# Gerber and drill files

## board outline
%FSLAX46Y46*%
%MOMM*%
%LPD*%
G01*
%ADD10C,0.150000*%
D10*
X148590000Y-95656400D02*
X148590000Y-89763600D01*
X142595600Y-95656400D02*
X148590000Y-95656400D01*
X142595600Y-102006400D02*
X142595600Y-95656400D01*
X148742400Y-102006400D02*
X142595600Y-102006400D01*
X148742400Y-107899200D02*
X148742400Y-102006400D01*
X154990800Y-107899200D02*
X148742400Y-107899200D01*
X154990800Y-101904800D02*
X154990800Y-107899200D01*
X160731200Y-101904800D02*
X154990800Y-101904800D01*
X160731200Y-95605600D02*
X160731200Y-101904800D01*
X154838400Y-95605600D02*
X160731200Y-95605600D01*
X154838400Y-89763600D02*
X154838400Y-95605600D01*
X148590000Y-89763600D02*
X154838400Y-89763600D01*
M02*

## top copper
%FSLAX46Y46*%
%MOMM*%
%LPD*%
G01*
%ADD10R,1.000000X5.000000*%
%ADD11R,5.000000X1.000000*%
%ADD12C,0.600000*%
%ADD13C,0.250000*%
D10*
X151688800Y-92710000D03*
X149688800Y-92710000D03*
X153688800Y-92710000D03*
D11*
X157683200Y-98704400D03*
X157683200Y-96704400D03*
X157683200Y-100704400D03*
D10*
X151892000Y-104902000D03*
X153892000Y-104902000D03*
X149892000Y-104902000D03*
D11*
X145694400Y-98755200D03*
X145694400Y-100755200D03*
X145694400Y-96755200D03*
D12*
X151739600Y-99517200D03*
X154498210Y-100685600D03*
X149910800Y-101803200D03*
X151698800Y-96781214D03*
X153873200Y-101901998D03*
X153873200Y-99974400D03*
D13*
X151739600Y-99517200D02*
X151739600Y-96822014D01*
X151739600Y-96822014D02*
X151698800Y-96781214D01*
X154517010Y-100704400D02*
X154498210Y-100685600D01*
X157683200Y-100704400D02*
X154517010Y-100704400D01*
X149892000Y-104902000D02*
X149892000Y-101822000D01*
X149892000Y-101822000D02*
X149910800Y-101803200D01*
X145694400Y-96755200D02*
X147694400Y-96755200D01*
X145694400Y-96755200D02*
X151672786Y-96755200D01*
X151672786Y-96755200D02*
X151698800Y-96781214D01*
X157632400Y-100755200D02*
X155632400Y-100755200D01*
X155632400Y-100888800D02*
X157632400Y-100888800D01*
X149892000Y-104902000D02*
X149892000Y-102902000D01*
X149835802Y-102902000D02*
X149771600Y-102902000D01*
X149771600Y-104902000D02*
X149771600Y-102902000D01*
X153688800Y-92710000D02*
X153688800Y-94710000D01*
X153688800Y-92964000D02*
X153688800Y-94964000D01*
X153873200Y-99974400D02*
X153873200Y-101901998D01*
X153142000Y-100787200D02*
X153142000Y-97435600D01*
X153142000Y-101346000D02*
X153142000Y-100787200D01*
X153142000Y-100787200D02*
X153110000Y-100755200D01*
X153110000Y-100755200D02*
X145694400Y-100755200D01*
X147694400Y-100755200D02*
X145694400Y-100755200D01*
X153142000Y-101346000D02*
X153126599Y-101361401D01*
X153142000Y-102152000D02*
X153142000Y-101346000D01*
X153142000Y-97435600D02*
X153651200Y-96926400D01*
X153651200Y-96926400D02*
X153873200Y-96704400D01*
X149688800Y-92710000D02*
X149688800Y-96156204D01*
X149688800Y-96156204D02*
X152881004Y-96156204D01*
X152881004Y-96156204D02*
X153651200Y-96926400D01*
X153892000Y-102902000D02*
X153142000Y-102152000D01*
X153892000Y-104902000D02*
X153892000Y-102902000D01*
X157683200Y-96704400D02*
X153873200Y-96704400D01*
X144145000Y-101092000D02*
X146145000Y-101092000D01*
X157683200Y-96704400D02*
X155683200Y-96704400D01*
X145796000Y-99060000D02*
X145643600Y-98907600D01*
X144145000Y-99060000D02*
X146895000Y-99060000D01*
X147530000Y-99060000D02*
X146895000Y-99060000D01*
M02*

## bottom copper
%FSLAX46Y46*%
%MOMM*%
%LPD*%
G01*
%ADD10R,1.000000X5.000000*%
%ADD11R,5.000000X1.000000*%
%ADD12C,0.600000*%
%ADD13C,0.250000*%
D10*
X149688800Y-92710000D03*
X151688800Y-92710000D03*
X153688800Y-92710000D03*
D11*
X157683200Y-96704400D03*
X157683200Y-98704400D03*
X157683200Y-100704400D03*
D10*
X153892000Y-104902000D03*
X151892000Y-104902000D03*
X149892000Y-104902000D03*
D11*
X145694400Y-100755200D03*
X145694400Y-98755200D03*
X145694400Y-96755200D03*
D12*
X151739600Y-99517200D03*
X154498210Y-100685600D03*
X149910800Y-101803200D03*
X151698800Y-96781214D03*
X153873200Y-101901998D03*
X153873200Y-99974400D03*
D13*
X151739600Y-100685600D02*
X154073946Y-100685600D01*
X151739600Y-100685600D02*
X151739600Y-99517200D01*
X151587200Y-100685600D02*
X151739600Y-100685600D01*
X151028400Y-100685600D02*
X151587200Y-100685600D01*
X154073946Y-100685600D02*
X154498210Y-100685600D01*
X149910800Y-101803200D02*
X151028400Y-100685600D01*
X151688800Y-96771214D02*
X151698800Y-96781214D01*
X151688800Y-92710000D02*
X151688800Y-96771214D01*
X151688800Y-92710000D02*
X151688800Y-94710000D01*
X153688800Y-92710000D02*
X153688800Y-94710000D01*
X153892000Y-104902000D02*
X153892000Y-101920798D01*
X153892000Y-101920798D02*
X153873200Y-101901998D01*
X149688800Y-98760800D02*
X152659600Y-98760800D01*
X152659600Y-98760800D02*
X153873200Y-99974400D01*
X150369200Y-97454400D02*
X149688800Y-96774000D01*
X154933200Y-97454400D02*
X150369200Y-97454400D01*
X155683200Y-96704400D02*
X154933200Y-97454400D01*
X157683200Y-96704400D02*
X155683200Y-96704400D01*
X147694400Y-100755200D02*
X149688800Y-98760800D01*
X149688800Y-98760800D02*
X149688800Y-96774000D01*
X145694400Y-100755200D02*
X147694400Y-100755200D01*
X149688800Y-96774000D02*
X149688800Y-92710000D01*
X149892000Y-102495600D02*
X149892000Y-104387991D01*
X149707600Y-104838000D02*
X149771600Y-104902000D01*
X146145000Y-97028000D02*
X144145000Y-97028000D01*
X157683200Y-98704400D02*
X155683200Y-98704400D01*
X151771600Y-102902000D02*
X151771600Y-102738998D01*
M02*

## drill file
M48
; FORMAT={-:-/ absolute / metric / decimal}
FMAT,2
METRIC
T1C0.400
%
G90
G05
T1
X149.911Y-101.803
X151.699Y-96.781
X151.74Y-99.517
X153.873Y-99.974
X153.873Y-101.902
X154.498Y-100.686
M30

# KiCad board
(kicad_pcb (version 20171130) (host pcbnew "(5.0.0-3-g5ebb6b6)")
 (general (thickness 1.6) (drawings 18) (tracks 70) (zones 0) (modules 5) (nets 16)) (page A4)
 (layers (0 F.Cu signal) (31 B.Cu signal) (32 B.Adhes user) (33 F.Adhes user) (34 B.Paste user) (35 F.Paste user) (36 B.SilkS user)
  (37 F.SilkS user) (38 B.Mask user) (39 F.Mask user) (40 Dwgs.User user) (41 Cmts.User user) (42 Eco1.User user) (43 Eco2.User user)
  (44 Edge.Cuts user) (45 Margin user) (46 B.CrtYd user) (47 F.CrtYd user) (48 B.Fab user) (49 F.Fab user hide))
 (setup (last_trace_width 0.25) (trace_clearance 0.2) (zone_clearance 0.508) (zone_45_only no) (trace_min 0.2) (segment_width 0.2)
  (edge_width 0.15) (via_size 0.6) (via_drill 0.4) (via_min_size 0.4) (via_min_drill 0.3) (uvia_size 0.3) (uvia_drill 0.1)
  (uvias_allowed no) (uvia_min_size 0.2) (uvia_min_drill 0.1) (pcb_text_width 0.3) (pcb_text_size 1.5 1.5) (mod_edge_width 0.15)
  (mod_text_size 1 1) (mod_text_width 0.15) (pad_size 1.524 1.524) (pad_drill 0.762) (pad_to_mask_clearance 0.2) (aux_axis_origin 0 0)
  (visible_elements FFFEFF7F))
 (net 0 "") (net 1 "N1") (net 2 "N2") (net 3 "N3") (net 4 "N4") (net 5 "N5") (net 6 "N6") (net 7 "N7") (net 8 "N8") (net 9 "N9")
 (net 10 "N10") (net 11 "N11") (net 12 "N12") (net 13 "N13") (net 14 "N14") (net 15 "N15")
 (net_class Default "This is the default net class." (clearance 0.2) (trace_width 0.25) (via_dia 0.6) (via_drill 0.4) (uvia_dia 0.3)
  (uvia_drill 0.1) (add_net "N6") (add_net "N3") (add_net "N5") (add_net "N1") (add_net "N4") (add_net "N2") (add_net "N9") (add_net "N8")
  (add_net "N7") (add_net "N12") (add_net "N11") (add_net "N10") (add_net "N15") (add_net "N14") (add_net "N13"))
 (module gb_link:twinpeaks (layer B.Cu) (at 149.86 100.33 180)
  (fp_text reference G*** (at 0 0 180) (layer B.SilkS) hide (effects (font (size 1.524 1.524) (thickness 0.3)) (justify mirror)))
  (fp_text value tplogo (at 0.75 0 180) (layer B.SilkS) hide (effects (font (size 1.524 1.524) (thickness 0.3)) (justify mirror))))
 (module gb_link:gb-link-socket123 (layer F.Cu) (at 151.6888 92.71 180)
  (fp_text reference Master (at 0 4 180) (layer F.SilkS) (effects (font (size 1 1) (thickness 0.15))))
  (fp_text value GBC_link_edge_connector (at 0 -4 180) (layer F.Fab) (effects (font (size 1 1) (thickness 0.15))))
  (pad 4 connect rect (at 0 0 180) (size 1 5) (layers F.Cu F.Mask) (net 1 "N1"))
  (pad 6 connect rect (at 2 0 180) (size 1 5) (layers F.Cu F.Mask) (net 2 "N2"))
  (pad 2 connect rect (at -2 0 180) (size 1 5) (layers F.Cu F.Mask) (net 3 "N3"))
  (pad 5 connect rect (at 2 0 180) (size 1 5) (layers B.Cu B.Mask) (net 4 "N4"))
  (pad 3 connect rect (at 0 0 180) (size 1 5) (layers B.Cu B.Mask) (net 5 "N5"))
  (pad 1 connect rect (at -2 0 180) (size 1 5) (layers B.Cu B.Mask) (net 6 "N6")))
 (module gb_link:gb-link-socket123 (layer F.Cu) (at 157.6832 98.7044 90)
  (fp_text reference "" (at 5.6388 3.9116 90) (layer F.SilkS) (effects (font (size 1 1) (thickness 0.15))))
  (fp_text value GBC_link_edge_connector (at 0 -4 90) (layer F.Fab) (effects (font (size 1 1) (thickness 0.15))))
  (pad 4 connect rect (at 0 0 90) (size 1 5) (layers F.Cu F.Mask) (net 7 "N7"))
  (pad 6 connect rect (at 2 0 90) (size 1 5) (layers F.Cu F.Mask) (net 2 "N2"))
  (pad 2 connect rect (at -2 0 90) (size 1 5) (layers F.Cu F.Mask) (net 5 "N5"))
  (pad 5 connect rect (at 2 0 90) (size 1 5) (layers B.Cu B.Mask) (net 4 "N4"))
  (pad 3 connect rect (at 0 0 90) (size 1 5) (layers B.Cu B.Mask) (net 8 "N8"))
  (pad 1 connect rect (at -2 0 90) (size 1 5) (layers B.Cu B.Mask) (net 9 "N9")))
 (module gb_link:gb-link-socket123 (layer F.Cu) (at 151.892 104.902)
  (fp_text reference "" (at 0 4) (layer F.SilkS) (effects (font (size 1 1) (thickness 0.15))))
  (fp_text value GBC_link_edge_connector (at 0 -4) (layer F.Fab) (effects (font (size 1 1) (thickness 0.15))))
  (pad 4 connect rect (at 0 0) (size 1 5) (layers F.Cu F.Mask) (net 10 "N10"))
  (pad 6 connect rect (at 2 0) (size 1 5) (layers F.Cu F.Mask) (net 2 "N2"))
  (pad 2 connect rect (at -2 0) (size 1 5) (layers F.Cu F.Mask) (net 5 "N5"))
  (pad 5 connect rect (at 2 0) (size 1 5) (layers B.Cu B.Mask) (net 4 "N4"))
  (pad 3 connect rect (at 0 0) (size 1 5) (layers B.Cu B.Mask) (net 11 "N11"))
  (pad 1 connect rect (at -2 0) (size 1 5) (layers B.Cu B.Mask) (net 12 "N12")))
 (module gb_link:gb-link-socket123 (layer F.Cu) (at 145.6944 98.7552 270)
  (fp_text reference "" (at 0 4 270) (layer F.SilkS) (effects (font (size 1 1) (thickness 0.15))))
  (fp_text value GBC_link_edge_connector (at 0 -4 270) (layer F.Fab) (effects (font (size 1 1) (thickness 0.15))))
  (pad 4 connect rect (at 0 0 270) (size 1 5) (layers F.Cu F.Mask) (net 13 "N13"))
  (pad 6 connect rect (at 2 0 270) (size 1 5) (layers F.Cu F.Mask) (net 2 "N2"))
  (pad 2 connect rect (at -2 0 270) (size 1 5) (layers F.Cu F.Mask) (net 5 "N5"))
  (pad 5 connect rect (at 2 0 270) (size 1 5) (layers B.Cu B.Mask) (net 4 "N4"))
  (pad 3 connect rect (at 0 0 270) (size 1 5) (layers B.Cu B.Mask) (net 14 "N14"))
  (pad 1 connect rect (at -2 0 270) (size 1 5) (layers B.Cu B.Mask) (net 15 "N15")))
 (gr_line (start 148.59 95.6564) (end 148.59 89.7636) (layer Edge.Cuts) (width 0.15))
 (gr_line (start 142.5956 95.6564) (end 148.59 95.6564) (layer Edge.Cuts) (width 0.15))
 (gr_line (start 142.5956 102.0064) (end 142.5956 95.6564) (layer Edge.Cuts) (width 0.15))
 (gr_line (start 148.7424 102.0064) (end 142.5956 102.0064) (layer Edge.Cuts) (width 0.15))
 (gr_line (start 148.7424 107.8992) (end 148.7424 102.0064) (layer Edge.Cuts) (width 0.15))
 (gr_line (start 154.9908 107.8992) (end 148.7424 107.8992) (layer Edge.Cuts) (width 0.15))
 (gr_line (start 154.9908 101.9048) (end 154.9908 107.8992) (layer Edge.Cuts) (width 0.15))
 (gr_line (start 160.7312 101.9048) (end 154.9908 101.9048) (layer Edge.Cuts) (width 0.15))
 (gr_line (start 160.7312 95.6056) (end 160.7312 101.9048) (layer Edge.Cuts) (width 0.15))
 (gr_line (start 154.8384 95.6056) (end 160.7312 95.6056) (layer Edge.Cuts) (width 0.15))
 (gr_line (start 154.8384 89.7636) (end 154.8384 95.6056) (layer Edge.Cuts) (width 0.15))
 (gr_line (start 148.59 89.7636) (end 154.8384 89.7636) (layer Edge.Cuts) (width 0.15))
 (segment (start 151.7396 99.5172) (end 151.7396 96.822014) (width 0.25) (layer F.Cu) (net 5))
 (segment (start 151.7396 96.822014) (end 151.6988 96.781214) (width 0.25) (layer F.Cu) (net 5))
 (segment (start 151.7396 100.6856) (end 154.073946 100.6856) (width 0.25) (layer B.Cu) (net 5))
 (segment (start 151.7396 100.6856) (end 151.7396 99.5172) (width 0.25) (layer B.Cu) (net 5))
 (segment (start 151.5872 100.6856) (end 151.7396 100.6856) (width 0.25) (layer B.Cu) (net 5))
 (via (at 151.7396 99.5172) (size 0.6) (drill 0.4) (layers F.Cu B.Cu) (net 5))
 (segment (start 151.0284 100.6856) (end 151.5872 100.6856) (width 0.25) (layer B.Cu) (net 5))
 (segment (start 154.073946 100.6856) (end 154.49821 100.6856) (width 0.25) (layer B.Cu) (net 5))
 (segment (start 149.9108 101.8032) (end 151.0284 100.6856) (width 0.25) (layer B.Cu) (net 5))
 (segment (start 154.51701 100.7044) (end 154.49821 100.6856) (width 0.25) (layer F.Cu) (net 5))
 (segment (start 157.6832 100.7044) (end 154.51701 100.7044) (width 0.25) (layer F.Cu) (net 5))
 (via (at 154.49821 100.6856) (size 0.6) (drill 0.4) (layers F.Cu B.Cu) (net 5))
 (segment (start 149.892 104.902) (end 149.892 101.822) (width 0.25) (layer F.Cu) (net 5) (status 10))
 (segment (start 149.892 101.822) (end 149.9108 101.8032) (width 0.25) (layer F.Cu) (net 5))
 (via (at 149.9108 101.8032) (size 0.6) (drill 0.4) (layers F.Cu B.Cu) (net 5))
 (segment (start 145.6944 96.7552) (end 147.6944 96.7552) (width 0.25) (layer F.Cu) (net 5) (status 30))
 (segment (start 145.6944 96.7552) (end 151.672786 96.7552) (width 0.25) (layer F.Cu) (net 5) (status 10))
 (segment (start 151.6888 96.771214) (end 151.6988 96.781214) (width 0.25) (layer B.Cu) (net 5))
 (segment (start 151.6888 92.71) (end 151.6888 96.771214) (width 0.25) (layer B.Cu) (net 5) (status 10))
 (segment (start 151.672786 96.7552) (end 151.6988 96.781214) (width 0.25) (layer F.Cu) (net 5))
 (via (at 151.6988 96.781214) (size 0.6) (drill 0.4) (layers F.Cu B.Cu) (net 5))
 (segment (start 151.6888 92.71) (end 151.6888 94.71) (width 0.25) (layer B.Cu) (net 5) (status 30))
 (segment (start 157.6324 100.7552) (end 155.6324 100.7552) (width 0.25) (layer F.Cu) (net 5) (status 30))
 (segment (start 155.6324 100.8888) (end 157.6324 100.8888) (width 0.25) (layer F.Cu) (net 5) (status 30))
 (segment (start 149.892 104.902) (end 149.892 102.902) (width 0.25) (layer F.Cu) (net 5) (status 30))
 (segment (start 149.835802 102.902) (end 149.7716 102.902) (width 0.25) (layer F.Cu) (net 5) (status 30))
 (segment (start 149.7716 104.902) (end 149.7716 102.902) (width 0.25) (layer F.Cu) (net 5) (status 30))
 (segment (start 153.6888 92.71) (end 153.6888 94.71) (width 0.25) (layer B.Cu) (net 6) (status 30))
 (segment (start 153.6888 92.71) (end 153.6888 94.71) (width 0.25) (layer F.Cu) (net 3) (status 30))
 (segment (start 153.6888 92.964) (end 153.6888 94.964) (width 0.25) (layer F.Cu) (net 3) (status 30))
 (segment (start 153.892 104.902) (end 153.892 101.920798) (width 0.25) (layer B.Cu) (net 4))
 (segment (start 153.892 101.920798) (end 153.8732 101.901998) (width 0.25) (layer B.Cu) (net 4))
 (segment (start 153.8732 99.9744) (end 153.8732 101.901998) (width 0.25) (layer F.Cu) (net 4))
 (via (at 153.8732 101.901998) (size 0.6) (drill 0.4) (layers F.Cu B.Cu) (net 4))
 (via (at 153.8732 99.9744) (size 0.6) (drill 0.4) (layers F.Cu B.Cu) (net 4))
 (segment (start 149.6888 98.7608) (end 152.6596 98.7608) (width 0.25) (layer B.Cu) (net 4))
 (segment (start 152.6596 98.7608) (end 153.8732 99.9744) (width 0.25) (layer B.Cu) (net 4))
 (segment (start 150.3692 97.4544) (end 149.6888 96.774) (width 0.25) (layer B.Cu) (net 4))
 (segment (start 154.9332 97.4544) (end 150.3692 97.4544) (width 0.25) (layer B.Cu) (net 4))
 (segment (start 155.6832 96.7044) (end 154.9332 97.4544) (width 0.25) (layer B.Cu) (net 4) (status 10))
 (segment (start 157.6832 96.7044) (end 155.6832 96.7044) (width 0.25) (layer B.Cu) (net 4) (status 30))
 (segment (start 147.6944 100.7552) (end 149.6888 98.7608) (width 0.25) (layer B.Cu) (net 4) (status 10))
 (segment (start 149.6888 98.7608) (end 149.6888 96.774) (width 0.25) (layer B.Cu) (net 4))
 (segment (start 145.6944 100.7552) (end 147.6944 100.7552) (width 0.25) (layer B.Cu) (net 4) (status 30))
 (segment (start 149.6888 96.774) (end 149.6888 92.71) (width 0.25) (layer B.Cu) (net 4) (status 20))
 (segment (start 153.142 100.7872) (end 153.142 97.4356) (width 0.25) (layer F.Cu) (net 2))
 (segment (start 153.142 101.346) (end 153.142 100.7872) (width 0.25) (layer F.Cu) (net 2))
 (segment (start 153.142 100.7872) (end 153.11 100.7552) (width 0.25) (layer F.Cu) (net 2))
 (segment (start 153.11 100.7552) (end 145.6944 100.7552) (width 0.25) (layer F.Cu) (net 2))
 (segment (start 147.6944 100.7552) (end 145.6944 100.7552) (width 0.25) (layer F.Cu) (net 2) (status 30))
 (segment (start 153.142 101.346) (end 153.126599 101.361401) (width 0.25) (layer F.Cu) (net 2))
 (segment (start 153.142 102.152) (end 153.142 101.346) (width 0.25) (layer F.Cu) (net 2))
 (segment (start 153.142 97.4356) (end 153.6512 96.9264) (width 0.25) (layer F.Cu) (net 2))
 (segment (start 153.6512 96.9264) (end 153.8732 96.7044) (width 0.25) (layer F.Cu) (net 2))
 (segment (start 149.6888 92.71) (end 149.6888 96.156204) (width 0.25) (layer F.Cu) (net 2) (status 10))
 (segment (start 149.6888 96.156204) (end 152.881004 96.156204) (width 0.25) (layer F.Cu) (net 2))
 (segment (start 152.881004 96.156204) (end 153.6512 96.9264) (width 0.25) (layer F.Cu) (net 2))
 (segment (start 153.892 102.902) (end 153.142 102.152) (width 0.25) (layer F.Cu) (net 2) (status 10))
 (segment (start 153.892 104.902) (end 153.892 102.902) (width 0.25) (layer F.Cu) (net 2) (status 30))
 (segment (start 157.6832 96.7044) (end 153.8732 96.7044) (width 0.25) (layer F.Cu) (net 2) (status 10))
 (segment (start 144.145 101.092) (end 146.145 101.092) (width 0.25) (layer F.Cu) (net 2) (status 30))
 (segment (start 157.6832 96.7044) (end 155.6832 96.7044) (width 0.25) (layer F.Cu) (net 2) (status 30))
 (segment (start 149.892 102.4956) (end 149.892 104.387991) (width 0.25) (layer B.Cu) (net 12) (status 30))
 (segment (start 149.7076 104.838) (end 149.7716 104.902) (width 0.25) (layer B.Cu) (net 12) (status 30))
 (segment (start 146.145 97.028) (end 144.145 97.028) (width 0.25) (layer B.Cu) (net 15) (status 30))
 (segment (start 145.796 99.06) (end 145.6436 98.9076) (width 0.25) (layer F.Cu) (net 13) (status 30))
 (segment (start 144.145 99.06) (end 146.895 99.06) (width 0.25) (layer F.Cu) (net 13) (status 30))
 (segment (start 147.53 99.06) (end 146.895 99.06) (width 0.25) (layer F.Cu) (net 13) (status 30))
 (segment (start 157.6832 98.7044) (end 155.6832 98.7044) (width 0.25) (layer B.Cu) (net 8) (status 30))
 (segment (start 151.7716 102.902) (end 151.7716 102.738998) (width 0.25) (layer B.Cu) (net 11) (status 30)))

